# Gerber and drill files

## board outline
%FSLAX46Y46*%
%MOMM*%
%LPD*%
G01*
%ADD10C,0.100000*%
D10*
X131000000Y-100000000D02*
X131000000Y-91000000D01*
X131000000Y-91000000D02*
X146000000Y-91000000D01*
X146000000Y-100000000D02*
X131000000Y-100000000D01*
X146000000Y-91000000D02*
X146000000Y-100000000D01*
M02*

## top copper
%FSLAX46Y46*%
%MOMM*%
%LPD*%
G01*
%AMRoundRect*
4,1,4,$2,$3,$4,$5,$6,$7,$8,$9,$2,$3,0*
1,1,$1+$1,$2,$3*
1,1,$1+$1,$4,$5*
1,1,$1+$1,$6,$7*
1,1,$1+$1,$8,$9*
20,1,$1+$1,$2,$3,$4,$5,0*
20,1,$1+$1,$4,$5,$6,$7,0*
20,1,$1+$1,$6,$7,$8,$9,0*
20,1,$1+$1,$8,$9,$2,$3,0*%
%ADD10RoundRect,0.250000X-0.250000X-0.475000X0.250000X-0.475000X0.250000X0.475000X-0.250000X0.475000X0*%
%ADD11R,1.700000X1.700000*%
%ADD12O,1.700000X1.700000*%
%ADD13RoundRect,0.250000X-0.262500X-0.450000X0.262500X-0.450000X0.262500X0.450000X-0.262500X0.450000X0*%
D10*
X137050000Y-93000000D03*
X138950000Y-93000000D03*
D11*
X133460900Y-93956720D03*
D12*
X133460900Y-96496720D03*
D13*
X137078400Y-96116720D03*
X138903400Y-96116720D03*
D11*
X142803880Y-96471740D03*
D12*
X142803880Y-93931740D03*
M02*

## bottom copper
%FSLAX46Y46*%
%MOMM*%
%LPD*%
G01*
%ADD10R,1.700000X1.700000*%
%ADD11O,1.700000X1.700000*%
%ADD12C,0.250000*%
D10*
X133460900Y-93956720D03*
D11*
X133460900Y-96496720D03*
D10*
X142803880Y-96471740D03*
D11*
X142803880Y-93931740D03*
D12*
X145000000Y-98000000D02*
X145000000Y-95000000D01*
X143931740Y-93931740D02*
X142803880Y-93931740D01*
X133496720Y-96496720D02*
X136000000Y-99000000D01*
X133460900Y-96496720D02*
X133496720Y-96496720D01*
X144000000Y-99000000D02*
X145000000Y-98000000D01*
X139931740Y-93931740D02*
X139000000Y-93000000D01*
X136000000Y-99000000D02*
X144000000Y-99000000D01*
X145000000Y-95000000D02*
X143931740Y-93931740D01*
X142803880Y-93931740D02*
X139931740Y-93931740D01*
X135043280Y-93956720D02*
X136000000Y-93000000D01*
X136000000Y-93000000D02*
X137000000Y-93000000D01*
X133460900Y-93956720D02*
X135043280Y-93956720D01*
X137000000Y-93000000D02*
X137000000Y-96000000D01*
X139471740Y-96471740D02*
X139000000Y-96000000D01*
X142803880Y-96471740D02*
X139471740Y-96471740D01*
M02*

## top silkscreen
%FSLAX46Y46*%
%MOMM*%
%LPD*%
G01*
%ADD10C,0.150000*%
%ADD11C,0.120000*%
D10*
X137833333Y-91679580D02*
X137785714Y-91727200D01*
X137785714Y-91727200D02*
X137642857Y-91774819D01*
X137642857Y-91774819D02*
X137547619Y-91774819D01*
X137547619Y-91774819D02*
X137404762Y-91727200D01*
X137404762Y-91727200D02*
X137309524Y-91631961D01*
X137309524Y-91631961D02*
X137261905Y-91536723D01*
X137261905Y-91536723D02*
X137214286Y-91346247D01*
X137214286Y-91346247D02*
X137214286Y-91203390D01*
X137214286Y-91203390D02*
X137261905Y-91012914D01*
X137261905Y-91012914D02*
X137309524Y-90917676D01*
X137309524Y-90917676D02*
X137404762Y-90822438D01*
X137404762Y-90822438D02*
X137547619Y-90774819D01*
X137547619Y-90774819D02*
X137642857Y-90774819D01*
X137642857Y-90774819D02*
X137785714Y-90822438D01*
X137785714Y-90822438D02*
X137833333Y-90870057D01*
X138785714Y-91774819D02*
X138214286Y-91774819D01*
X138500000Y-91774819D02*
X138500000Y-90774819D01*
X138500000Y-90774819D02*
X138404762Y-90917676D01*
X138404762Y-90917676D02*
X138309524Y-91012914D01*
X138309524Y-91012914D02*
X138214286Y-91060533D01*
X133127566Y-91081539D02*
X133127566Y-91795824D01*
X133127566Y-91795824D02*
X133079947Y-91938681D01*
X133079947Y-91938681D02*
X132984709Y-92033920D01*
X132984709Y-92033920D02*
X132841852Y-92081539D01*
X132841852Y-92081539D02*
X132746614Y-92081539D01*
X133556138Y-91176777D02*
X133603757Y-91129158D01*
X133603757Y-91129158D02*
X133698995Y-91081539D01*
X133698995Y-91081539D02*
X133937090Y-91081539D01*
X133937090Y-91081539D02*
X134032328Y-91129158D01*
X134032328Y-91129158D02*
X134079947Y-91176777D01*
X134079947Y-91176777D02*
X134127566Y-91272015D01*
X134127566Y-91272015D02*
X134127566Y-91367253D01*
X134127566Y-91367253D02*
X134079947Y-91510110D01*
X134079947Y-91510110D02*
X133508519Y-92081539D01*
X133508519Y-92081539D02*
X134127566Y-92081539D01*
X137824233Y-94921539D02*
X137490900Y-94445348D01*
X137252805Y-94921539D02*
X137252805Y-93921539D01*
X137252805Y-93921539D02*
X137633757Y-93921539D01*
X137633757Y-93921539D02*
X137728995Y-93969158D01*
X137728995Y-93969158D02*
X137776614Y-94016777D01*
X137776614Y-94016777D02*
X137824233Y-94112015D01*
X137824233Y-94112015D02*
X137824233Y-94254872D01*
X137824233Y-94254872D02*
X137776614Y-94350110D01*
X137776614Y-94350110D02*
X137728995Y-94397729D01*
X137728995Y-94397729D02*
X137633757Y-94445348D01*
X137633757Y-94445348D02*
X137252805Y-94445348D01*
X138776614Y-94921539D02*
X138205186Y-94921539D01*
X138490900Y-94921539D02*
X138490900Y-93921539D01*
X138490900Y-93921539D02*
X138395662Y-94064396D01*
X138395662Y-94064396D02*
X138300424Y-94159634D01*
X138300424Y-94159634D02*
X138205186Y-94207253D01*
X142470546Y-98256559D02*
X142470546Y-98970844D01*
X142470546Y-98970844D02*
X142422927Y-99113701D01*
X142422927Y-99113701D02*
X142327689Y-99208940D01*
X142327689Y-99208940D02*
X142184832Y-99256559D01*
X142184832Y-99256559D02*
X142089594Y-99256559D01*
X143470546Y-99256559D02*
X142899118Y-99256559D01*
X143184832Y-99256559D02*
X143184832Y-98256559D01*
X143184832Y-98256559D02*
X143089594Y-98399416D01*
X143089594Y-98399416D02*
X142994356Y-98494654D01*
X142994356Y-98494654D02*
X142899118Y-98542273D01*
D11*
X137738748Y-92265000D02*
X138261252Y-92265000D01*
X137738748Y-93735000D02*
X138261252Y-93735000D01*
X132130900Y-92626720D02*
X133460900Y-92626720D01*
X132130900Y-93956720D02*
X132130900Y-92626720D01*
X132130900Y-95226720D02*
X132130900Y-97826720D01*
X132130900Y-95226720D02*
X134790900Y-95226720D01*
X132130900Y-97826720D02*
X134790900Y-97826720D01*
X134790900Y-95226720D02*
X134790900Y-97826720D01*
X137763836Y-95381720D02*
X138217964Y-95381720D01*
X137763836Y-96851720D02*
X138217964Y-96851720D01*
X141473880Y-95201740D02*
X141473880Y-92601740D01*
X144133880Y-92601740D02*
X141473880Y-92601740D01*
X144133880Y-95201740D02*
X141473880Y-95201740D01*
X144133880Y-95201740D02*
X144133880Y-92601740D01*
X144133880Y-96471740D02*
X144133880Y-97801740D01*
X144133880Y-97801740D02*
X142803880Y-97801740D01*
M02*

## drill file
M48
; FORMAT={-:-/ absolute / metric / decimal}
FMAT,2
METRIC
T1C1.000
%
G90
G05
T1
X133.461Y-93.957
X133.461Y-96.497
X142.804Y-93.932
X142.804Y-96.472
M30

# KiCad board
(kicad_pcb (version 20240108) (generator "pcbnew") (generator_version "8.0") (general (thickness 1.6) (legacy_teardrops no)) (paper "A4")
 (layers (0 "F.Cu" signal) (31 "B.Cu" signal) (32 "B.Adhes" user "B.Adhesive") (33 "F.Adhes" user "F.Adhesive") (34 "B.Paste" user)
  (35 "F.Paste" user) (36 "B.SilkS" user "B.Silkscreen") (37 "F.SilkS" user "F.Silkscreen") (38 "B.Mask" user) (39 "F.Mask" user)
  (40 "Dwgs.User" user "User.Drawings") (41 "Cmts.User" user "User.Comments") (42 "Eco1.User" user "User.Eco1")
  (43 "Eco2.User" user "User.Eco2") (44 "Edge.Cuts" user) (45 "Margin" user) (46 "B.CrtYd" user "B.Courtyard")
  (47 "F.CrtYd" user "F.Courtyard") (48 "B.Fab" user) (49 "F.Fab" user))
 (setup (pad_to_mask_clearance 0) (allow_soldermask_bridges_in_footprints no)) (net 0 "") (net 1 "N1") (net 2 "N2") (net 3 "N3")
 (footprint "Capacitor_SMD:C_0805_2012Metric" (layer "F.Cu") (at 138 93)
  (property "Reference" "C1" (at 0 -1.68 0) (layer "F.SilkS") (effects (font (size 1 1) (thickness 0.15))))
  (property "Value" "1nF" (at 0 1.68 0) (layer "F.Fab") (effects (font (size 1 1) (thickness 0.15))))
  (fp_line (start -0.261252 -0.735) (end 0.261252 -0.735) (stroke (width 0.12) (type solid)) (layer "F.SilkS"))
  (fp_line (start -0.261252 0.735) (end 0.261252 0.735) (stroke (width 0.12) (type solid)) (layer "F.SilkS"))
  (pad "1" smd roundrect (at -0.95 0) (size 1 1.45) (layers "F.Cu" "F.Paste" "F.Mask") (roundrect_rratio 0.25) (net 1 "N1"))
  (pad "2" smd roundrect (at 0.95 0) (size 1 1.45) (layers "F.Cu" "F.Paste" "F.Mask") (roundrect_rratio 0.25) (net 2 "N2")))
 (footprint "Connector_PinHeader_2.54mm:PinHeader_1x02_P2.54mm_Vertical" (layer "F.Cu") (at 133.4609 93.95672)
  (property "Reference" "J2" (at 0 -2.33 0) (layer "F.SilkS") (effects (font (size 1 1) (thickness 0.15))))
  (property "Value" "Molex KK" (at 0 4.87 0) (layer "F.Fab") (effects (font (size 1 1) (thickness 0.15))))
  (fp_line (start -1.33 -1.33) (end 0 -1.33) (stroke (width 0.12) (type solid)) (layer "F.SilkS"))
  (fp_line (start -1.33 0) (end -1.33 -1.33) (stroke (width 0.12) (type solid)) (layer "F.SilkS"))
  (fp_line (start -1.33 1.27) (end -1.33 3.87) (stroke (width 0.12) (type solid)) (layer "F.SilkS"))
  (fp_line (start -1.33 1.27) (end 1.33 1.27) (stroke (width 0.12) (type solid)) (layer "F.SilkS"))
  (fp_line (start -1.33 3.87) (end 1.33 3.87) (stroke (width 0.12) (type solid)) (layer "F.SilkS"))
  (fp_line (start 1.33 1.27) (end 1.33 3.87) (stroke (width 0.12) (type solid)) (layer "F.SilkS"))
  (pad "1" thru_hole rect (at 0 0) (size 1.7 1.7) (drill 1) (layers "*.Cu" "*.Mask") (remove_unused_layers no) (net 1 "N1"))
  (pad "2" thru_hole oval (at 0 2.54) (size 1.7 1.7) (drill 1) (layers "*.Cu" "*.Mask") (remove_unused_layers no) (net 2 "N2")))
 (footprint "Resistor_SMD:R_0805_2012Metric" (layer "F.Cu") (at 137.9909 96.11672)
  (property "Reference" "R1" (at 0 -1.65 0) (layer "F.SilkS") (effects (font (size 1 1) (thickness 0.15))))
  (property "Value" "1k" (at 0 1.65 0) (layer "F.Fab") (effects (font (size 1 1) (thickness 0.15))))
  (fp_line (start -0.227064 -0.735) (end 0.227064 -0.735) (stroke (width 0.12) (type solid)) (layer "F.SilkS"))
  (fp_line (start -0.227064 0.735) (end 0.227064 0.735) (stroke (width 0.12) (type solid)) (layer "F.SilkS"))
  (pad "1" smd roundrect (at -0.9125 0) (size 1.025 1.4) (layers "F.Cu" "F.Paste" "F.Mask") (roundrect_rratio 0.243902) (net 1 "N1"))
  (pad "2" smd roundrect (at 0.9125 0) (size 1.025 1.4) (layers "F.Cu" "F.Paste" "F.Mask") (roundrect_rratio 0.243902) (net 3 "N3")))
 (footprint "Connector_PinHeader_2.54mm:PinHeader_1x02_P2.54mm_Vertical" (layer "F.Cu") (at 142.80388 96.47174 180)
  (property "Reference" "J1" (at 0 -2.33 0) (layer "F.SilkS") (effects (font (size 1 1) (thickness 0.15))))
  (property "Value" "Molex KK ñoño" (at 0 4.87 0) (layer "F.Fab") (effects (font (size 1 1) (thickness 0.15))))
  (fp_line (start 1.33 1.27) (end 1.33 3.87) (stroke (width 0.12) (type solid)) (layer "F.SilkS"))
  (fp_line (start -1.33 3.87) (end 1.33 3.87) (stroke (width 0.12) (type solid)) (layer "F.SilkS"))
  (fp_line (start -1.33 1.27) (end 1.33 1.27) (stroke (width 0.12) (type solid)) (layer "F.SilkS"))
  (fp_line (start -1.33 1.27) (end -1.33 3.87) (stroke (width 0.12) (type solid)) (layer "F.SilkS"))
  (fp_line (start -1.33 0) (end -1.33 -1.33) (stroke (width 0.12) (type solid)) (layer "F.SilkS"))
  (fp_line (start -1.33 -1.33) (end 0 -1.33) (stroke (width 0.12) (type solid)) (layer "F.SilkS"))
  (pad "1" thru_hole rect (at 0 0 180) (size 1.7 1.7) (drill 1) (layers "*.Cu" "*.Mask") (remove_unused_layers no) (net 3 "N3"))
  (pad "2" thru_hole oval (at 0 2.54 180) (size 1.7 1.7) (drill 1) (layers "*.Cu" "*.Mask") (remove_unused_layers no) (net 2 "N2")))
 (gr_line (start 131 100) (end 131 91) (stroke (width 0.1) (type solid)) (layer "Edge.Cuts"))
 (gr_line (start 131 91) (end 146 91) (stroke (width 0.1) (type solid)) (layer "Edge.Cuts"))
 (gr_line (start 146 100) (end 131 100) (stroke (width 0.1) (type solid)) (layer "Edge.Cuts"))
 (gr_line (start 146 91) (end 146 100) (stroke (width 0.1) (type solid)) (layer "Edge.Cuts"))
 (segment (start 145 98) (end 145 95) (width 0.25) (layer "B.Cu") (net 2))
 (segment (start 143.93174 93.93174) (end 142.80388 93.93174) (width 0.25) (layer "B.Cu") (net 2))
 (segment (start 133.49672 96.49672) (end 136 99) (width 0.25) (layer "B.Cu") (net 2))
 (segment (start 133.4609 96.49672) (end 133.49672 96.49672) (width 0.25) (layer "B.Cu") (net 2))
 (segment (start 144 99) (end 145 98) (width 0.25) (layer "B.Cu") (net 2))
 (segment (start 139.93174 93.93174) (end 139 93) (width 0.25) (layer "B.Cu") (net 2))
 (segment (start 136 99) (end 144 99) (width 0.25) (layer "B.Cu") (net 2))
 (segment (start 145 95) (end 143.93174 93.93174) (width 0.25) (layer "B.Cu") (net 2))
 (segment (start 142.80388 93.93174) (end 139.93174 93.93174) (width 0.25) (layer "B.Cu") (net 2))
 (segment (start 135.04328 93.95672) (end 136 93) (width 0.25) (layer "B.Cu") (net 1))
 (segment (start 136 93) (end 137 93) (width 0.25) (layer "B.Cu") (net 1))
 (segment (start 133.4609 93.95672) (end 135.04328 93.95672) (width 0.25) (layer "B.Cu") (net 1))
 (segment (start 137 93) (end 137 96) (width 0.25) (layer "B.Cu") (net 1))
 (segment (start 139.47174 96.47174) (end 139 96) (width 0.25) (layer "B.Cu") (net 3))
 (segment (start 142.80388 96.47174) (end 139.47174 96.47174) (width 0.25) (layer "B.Cu") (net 3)))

